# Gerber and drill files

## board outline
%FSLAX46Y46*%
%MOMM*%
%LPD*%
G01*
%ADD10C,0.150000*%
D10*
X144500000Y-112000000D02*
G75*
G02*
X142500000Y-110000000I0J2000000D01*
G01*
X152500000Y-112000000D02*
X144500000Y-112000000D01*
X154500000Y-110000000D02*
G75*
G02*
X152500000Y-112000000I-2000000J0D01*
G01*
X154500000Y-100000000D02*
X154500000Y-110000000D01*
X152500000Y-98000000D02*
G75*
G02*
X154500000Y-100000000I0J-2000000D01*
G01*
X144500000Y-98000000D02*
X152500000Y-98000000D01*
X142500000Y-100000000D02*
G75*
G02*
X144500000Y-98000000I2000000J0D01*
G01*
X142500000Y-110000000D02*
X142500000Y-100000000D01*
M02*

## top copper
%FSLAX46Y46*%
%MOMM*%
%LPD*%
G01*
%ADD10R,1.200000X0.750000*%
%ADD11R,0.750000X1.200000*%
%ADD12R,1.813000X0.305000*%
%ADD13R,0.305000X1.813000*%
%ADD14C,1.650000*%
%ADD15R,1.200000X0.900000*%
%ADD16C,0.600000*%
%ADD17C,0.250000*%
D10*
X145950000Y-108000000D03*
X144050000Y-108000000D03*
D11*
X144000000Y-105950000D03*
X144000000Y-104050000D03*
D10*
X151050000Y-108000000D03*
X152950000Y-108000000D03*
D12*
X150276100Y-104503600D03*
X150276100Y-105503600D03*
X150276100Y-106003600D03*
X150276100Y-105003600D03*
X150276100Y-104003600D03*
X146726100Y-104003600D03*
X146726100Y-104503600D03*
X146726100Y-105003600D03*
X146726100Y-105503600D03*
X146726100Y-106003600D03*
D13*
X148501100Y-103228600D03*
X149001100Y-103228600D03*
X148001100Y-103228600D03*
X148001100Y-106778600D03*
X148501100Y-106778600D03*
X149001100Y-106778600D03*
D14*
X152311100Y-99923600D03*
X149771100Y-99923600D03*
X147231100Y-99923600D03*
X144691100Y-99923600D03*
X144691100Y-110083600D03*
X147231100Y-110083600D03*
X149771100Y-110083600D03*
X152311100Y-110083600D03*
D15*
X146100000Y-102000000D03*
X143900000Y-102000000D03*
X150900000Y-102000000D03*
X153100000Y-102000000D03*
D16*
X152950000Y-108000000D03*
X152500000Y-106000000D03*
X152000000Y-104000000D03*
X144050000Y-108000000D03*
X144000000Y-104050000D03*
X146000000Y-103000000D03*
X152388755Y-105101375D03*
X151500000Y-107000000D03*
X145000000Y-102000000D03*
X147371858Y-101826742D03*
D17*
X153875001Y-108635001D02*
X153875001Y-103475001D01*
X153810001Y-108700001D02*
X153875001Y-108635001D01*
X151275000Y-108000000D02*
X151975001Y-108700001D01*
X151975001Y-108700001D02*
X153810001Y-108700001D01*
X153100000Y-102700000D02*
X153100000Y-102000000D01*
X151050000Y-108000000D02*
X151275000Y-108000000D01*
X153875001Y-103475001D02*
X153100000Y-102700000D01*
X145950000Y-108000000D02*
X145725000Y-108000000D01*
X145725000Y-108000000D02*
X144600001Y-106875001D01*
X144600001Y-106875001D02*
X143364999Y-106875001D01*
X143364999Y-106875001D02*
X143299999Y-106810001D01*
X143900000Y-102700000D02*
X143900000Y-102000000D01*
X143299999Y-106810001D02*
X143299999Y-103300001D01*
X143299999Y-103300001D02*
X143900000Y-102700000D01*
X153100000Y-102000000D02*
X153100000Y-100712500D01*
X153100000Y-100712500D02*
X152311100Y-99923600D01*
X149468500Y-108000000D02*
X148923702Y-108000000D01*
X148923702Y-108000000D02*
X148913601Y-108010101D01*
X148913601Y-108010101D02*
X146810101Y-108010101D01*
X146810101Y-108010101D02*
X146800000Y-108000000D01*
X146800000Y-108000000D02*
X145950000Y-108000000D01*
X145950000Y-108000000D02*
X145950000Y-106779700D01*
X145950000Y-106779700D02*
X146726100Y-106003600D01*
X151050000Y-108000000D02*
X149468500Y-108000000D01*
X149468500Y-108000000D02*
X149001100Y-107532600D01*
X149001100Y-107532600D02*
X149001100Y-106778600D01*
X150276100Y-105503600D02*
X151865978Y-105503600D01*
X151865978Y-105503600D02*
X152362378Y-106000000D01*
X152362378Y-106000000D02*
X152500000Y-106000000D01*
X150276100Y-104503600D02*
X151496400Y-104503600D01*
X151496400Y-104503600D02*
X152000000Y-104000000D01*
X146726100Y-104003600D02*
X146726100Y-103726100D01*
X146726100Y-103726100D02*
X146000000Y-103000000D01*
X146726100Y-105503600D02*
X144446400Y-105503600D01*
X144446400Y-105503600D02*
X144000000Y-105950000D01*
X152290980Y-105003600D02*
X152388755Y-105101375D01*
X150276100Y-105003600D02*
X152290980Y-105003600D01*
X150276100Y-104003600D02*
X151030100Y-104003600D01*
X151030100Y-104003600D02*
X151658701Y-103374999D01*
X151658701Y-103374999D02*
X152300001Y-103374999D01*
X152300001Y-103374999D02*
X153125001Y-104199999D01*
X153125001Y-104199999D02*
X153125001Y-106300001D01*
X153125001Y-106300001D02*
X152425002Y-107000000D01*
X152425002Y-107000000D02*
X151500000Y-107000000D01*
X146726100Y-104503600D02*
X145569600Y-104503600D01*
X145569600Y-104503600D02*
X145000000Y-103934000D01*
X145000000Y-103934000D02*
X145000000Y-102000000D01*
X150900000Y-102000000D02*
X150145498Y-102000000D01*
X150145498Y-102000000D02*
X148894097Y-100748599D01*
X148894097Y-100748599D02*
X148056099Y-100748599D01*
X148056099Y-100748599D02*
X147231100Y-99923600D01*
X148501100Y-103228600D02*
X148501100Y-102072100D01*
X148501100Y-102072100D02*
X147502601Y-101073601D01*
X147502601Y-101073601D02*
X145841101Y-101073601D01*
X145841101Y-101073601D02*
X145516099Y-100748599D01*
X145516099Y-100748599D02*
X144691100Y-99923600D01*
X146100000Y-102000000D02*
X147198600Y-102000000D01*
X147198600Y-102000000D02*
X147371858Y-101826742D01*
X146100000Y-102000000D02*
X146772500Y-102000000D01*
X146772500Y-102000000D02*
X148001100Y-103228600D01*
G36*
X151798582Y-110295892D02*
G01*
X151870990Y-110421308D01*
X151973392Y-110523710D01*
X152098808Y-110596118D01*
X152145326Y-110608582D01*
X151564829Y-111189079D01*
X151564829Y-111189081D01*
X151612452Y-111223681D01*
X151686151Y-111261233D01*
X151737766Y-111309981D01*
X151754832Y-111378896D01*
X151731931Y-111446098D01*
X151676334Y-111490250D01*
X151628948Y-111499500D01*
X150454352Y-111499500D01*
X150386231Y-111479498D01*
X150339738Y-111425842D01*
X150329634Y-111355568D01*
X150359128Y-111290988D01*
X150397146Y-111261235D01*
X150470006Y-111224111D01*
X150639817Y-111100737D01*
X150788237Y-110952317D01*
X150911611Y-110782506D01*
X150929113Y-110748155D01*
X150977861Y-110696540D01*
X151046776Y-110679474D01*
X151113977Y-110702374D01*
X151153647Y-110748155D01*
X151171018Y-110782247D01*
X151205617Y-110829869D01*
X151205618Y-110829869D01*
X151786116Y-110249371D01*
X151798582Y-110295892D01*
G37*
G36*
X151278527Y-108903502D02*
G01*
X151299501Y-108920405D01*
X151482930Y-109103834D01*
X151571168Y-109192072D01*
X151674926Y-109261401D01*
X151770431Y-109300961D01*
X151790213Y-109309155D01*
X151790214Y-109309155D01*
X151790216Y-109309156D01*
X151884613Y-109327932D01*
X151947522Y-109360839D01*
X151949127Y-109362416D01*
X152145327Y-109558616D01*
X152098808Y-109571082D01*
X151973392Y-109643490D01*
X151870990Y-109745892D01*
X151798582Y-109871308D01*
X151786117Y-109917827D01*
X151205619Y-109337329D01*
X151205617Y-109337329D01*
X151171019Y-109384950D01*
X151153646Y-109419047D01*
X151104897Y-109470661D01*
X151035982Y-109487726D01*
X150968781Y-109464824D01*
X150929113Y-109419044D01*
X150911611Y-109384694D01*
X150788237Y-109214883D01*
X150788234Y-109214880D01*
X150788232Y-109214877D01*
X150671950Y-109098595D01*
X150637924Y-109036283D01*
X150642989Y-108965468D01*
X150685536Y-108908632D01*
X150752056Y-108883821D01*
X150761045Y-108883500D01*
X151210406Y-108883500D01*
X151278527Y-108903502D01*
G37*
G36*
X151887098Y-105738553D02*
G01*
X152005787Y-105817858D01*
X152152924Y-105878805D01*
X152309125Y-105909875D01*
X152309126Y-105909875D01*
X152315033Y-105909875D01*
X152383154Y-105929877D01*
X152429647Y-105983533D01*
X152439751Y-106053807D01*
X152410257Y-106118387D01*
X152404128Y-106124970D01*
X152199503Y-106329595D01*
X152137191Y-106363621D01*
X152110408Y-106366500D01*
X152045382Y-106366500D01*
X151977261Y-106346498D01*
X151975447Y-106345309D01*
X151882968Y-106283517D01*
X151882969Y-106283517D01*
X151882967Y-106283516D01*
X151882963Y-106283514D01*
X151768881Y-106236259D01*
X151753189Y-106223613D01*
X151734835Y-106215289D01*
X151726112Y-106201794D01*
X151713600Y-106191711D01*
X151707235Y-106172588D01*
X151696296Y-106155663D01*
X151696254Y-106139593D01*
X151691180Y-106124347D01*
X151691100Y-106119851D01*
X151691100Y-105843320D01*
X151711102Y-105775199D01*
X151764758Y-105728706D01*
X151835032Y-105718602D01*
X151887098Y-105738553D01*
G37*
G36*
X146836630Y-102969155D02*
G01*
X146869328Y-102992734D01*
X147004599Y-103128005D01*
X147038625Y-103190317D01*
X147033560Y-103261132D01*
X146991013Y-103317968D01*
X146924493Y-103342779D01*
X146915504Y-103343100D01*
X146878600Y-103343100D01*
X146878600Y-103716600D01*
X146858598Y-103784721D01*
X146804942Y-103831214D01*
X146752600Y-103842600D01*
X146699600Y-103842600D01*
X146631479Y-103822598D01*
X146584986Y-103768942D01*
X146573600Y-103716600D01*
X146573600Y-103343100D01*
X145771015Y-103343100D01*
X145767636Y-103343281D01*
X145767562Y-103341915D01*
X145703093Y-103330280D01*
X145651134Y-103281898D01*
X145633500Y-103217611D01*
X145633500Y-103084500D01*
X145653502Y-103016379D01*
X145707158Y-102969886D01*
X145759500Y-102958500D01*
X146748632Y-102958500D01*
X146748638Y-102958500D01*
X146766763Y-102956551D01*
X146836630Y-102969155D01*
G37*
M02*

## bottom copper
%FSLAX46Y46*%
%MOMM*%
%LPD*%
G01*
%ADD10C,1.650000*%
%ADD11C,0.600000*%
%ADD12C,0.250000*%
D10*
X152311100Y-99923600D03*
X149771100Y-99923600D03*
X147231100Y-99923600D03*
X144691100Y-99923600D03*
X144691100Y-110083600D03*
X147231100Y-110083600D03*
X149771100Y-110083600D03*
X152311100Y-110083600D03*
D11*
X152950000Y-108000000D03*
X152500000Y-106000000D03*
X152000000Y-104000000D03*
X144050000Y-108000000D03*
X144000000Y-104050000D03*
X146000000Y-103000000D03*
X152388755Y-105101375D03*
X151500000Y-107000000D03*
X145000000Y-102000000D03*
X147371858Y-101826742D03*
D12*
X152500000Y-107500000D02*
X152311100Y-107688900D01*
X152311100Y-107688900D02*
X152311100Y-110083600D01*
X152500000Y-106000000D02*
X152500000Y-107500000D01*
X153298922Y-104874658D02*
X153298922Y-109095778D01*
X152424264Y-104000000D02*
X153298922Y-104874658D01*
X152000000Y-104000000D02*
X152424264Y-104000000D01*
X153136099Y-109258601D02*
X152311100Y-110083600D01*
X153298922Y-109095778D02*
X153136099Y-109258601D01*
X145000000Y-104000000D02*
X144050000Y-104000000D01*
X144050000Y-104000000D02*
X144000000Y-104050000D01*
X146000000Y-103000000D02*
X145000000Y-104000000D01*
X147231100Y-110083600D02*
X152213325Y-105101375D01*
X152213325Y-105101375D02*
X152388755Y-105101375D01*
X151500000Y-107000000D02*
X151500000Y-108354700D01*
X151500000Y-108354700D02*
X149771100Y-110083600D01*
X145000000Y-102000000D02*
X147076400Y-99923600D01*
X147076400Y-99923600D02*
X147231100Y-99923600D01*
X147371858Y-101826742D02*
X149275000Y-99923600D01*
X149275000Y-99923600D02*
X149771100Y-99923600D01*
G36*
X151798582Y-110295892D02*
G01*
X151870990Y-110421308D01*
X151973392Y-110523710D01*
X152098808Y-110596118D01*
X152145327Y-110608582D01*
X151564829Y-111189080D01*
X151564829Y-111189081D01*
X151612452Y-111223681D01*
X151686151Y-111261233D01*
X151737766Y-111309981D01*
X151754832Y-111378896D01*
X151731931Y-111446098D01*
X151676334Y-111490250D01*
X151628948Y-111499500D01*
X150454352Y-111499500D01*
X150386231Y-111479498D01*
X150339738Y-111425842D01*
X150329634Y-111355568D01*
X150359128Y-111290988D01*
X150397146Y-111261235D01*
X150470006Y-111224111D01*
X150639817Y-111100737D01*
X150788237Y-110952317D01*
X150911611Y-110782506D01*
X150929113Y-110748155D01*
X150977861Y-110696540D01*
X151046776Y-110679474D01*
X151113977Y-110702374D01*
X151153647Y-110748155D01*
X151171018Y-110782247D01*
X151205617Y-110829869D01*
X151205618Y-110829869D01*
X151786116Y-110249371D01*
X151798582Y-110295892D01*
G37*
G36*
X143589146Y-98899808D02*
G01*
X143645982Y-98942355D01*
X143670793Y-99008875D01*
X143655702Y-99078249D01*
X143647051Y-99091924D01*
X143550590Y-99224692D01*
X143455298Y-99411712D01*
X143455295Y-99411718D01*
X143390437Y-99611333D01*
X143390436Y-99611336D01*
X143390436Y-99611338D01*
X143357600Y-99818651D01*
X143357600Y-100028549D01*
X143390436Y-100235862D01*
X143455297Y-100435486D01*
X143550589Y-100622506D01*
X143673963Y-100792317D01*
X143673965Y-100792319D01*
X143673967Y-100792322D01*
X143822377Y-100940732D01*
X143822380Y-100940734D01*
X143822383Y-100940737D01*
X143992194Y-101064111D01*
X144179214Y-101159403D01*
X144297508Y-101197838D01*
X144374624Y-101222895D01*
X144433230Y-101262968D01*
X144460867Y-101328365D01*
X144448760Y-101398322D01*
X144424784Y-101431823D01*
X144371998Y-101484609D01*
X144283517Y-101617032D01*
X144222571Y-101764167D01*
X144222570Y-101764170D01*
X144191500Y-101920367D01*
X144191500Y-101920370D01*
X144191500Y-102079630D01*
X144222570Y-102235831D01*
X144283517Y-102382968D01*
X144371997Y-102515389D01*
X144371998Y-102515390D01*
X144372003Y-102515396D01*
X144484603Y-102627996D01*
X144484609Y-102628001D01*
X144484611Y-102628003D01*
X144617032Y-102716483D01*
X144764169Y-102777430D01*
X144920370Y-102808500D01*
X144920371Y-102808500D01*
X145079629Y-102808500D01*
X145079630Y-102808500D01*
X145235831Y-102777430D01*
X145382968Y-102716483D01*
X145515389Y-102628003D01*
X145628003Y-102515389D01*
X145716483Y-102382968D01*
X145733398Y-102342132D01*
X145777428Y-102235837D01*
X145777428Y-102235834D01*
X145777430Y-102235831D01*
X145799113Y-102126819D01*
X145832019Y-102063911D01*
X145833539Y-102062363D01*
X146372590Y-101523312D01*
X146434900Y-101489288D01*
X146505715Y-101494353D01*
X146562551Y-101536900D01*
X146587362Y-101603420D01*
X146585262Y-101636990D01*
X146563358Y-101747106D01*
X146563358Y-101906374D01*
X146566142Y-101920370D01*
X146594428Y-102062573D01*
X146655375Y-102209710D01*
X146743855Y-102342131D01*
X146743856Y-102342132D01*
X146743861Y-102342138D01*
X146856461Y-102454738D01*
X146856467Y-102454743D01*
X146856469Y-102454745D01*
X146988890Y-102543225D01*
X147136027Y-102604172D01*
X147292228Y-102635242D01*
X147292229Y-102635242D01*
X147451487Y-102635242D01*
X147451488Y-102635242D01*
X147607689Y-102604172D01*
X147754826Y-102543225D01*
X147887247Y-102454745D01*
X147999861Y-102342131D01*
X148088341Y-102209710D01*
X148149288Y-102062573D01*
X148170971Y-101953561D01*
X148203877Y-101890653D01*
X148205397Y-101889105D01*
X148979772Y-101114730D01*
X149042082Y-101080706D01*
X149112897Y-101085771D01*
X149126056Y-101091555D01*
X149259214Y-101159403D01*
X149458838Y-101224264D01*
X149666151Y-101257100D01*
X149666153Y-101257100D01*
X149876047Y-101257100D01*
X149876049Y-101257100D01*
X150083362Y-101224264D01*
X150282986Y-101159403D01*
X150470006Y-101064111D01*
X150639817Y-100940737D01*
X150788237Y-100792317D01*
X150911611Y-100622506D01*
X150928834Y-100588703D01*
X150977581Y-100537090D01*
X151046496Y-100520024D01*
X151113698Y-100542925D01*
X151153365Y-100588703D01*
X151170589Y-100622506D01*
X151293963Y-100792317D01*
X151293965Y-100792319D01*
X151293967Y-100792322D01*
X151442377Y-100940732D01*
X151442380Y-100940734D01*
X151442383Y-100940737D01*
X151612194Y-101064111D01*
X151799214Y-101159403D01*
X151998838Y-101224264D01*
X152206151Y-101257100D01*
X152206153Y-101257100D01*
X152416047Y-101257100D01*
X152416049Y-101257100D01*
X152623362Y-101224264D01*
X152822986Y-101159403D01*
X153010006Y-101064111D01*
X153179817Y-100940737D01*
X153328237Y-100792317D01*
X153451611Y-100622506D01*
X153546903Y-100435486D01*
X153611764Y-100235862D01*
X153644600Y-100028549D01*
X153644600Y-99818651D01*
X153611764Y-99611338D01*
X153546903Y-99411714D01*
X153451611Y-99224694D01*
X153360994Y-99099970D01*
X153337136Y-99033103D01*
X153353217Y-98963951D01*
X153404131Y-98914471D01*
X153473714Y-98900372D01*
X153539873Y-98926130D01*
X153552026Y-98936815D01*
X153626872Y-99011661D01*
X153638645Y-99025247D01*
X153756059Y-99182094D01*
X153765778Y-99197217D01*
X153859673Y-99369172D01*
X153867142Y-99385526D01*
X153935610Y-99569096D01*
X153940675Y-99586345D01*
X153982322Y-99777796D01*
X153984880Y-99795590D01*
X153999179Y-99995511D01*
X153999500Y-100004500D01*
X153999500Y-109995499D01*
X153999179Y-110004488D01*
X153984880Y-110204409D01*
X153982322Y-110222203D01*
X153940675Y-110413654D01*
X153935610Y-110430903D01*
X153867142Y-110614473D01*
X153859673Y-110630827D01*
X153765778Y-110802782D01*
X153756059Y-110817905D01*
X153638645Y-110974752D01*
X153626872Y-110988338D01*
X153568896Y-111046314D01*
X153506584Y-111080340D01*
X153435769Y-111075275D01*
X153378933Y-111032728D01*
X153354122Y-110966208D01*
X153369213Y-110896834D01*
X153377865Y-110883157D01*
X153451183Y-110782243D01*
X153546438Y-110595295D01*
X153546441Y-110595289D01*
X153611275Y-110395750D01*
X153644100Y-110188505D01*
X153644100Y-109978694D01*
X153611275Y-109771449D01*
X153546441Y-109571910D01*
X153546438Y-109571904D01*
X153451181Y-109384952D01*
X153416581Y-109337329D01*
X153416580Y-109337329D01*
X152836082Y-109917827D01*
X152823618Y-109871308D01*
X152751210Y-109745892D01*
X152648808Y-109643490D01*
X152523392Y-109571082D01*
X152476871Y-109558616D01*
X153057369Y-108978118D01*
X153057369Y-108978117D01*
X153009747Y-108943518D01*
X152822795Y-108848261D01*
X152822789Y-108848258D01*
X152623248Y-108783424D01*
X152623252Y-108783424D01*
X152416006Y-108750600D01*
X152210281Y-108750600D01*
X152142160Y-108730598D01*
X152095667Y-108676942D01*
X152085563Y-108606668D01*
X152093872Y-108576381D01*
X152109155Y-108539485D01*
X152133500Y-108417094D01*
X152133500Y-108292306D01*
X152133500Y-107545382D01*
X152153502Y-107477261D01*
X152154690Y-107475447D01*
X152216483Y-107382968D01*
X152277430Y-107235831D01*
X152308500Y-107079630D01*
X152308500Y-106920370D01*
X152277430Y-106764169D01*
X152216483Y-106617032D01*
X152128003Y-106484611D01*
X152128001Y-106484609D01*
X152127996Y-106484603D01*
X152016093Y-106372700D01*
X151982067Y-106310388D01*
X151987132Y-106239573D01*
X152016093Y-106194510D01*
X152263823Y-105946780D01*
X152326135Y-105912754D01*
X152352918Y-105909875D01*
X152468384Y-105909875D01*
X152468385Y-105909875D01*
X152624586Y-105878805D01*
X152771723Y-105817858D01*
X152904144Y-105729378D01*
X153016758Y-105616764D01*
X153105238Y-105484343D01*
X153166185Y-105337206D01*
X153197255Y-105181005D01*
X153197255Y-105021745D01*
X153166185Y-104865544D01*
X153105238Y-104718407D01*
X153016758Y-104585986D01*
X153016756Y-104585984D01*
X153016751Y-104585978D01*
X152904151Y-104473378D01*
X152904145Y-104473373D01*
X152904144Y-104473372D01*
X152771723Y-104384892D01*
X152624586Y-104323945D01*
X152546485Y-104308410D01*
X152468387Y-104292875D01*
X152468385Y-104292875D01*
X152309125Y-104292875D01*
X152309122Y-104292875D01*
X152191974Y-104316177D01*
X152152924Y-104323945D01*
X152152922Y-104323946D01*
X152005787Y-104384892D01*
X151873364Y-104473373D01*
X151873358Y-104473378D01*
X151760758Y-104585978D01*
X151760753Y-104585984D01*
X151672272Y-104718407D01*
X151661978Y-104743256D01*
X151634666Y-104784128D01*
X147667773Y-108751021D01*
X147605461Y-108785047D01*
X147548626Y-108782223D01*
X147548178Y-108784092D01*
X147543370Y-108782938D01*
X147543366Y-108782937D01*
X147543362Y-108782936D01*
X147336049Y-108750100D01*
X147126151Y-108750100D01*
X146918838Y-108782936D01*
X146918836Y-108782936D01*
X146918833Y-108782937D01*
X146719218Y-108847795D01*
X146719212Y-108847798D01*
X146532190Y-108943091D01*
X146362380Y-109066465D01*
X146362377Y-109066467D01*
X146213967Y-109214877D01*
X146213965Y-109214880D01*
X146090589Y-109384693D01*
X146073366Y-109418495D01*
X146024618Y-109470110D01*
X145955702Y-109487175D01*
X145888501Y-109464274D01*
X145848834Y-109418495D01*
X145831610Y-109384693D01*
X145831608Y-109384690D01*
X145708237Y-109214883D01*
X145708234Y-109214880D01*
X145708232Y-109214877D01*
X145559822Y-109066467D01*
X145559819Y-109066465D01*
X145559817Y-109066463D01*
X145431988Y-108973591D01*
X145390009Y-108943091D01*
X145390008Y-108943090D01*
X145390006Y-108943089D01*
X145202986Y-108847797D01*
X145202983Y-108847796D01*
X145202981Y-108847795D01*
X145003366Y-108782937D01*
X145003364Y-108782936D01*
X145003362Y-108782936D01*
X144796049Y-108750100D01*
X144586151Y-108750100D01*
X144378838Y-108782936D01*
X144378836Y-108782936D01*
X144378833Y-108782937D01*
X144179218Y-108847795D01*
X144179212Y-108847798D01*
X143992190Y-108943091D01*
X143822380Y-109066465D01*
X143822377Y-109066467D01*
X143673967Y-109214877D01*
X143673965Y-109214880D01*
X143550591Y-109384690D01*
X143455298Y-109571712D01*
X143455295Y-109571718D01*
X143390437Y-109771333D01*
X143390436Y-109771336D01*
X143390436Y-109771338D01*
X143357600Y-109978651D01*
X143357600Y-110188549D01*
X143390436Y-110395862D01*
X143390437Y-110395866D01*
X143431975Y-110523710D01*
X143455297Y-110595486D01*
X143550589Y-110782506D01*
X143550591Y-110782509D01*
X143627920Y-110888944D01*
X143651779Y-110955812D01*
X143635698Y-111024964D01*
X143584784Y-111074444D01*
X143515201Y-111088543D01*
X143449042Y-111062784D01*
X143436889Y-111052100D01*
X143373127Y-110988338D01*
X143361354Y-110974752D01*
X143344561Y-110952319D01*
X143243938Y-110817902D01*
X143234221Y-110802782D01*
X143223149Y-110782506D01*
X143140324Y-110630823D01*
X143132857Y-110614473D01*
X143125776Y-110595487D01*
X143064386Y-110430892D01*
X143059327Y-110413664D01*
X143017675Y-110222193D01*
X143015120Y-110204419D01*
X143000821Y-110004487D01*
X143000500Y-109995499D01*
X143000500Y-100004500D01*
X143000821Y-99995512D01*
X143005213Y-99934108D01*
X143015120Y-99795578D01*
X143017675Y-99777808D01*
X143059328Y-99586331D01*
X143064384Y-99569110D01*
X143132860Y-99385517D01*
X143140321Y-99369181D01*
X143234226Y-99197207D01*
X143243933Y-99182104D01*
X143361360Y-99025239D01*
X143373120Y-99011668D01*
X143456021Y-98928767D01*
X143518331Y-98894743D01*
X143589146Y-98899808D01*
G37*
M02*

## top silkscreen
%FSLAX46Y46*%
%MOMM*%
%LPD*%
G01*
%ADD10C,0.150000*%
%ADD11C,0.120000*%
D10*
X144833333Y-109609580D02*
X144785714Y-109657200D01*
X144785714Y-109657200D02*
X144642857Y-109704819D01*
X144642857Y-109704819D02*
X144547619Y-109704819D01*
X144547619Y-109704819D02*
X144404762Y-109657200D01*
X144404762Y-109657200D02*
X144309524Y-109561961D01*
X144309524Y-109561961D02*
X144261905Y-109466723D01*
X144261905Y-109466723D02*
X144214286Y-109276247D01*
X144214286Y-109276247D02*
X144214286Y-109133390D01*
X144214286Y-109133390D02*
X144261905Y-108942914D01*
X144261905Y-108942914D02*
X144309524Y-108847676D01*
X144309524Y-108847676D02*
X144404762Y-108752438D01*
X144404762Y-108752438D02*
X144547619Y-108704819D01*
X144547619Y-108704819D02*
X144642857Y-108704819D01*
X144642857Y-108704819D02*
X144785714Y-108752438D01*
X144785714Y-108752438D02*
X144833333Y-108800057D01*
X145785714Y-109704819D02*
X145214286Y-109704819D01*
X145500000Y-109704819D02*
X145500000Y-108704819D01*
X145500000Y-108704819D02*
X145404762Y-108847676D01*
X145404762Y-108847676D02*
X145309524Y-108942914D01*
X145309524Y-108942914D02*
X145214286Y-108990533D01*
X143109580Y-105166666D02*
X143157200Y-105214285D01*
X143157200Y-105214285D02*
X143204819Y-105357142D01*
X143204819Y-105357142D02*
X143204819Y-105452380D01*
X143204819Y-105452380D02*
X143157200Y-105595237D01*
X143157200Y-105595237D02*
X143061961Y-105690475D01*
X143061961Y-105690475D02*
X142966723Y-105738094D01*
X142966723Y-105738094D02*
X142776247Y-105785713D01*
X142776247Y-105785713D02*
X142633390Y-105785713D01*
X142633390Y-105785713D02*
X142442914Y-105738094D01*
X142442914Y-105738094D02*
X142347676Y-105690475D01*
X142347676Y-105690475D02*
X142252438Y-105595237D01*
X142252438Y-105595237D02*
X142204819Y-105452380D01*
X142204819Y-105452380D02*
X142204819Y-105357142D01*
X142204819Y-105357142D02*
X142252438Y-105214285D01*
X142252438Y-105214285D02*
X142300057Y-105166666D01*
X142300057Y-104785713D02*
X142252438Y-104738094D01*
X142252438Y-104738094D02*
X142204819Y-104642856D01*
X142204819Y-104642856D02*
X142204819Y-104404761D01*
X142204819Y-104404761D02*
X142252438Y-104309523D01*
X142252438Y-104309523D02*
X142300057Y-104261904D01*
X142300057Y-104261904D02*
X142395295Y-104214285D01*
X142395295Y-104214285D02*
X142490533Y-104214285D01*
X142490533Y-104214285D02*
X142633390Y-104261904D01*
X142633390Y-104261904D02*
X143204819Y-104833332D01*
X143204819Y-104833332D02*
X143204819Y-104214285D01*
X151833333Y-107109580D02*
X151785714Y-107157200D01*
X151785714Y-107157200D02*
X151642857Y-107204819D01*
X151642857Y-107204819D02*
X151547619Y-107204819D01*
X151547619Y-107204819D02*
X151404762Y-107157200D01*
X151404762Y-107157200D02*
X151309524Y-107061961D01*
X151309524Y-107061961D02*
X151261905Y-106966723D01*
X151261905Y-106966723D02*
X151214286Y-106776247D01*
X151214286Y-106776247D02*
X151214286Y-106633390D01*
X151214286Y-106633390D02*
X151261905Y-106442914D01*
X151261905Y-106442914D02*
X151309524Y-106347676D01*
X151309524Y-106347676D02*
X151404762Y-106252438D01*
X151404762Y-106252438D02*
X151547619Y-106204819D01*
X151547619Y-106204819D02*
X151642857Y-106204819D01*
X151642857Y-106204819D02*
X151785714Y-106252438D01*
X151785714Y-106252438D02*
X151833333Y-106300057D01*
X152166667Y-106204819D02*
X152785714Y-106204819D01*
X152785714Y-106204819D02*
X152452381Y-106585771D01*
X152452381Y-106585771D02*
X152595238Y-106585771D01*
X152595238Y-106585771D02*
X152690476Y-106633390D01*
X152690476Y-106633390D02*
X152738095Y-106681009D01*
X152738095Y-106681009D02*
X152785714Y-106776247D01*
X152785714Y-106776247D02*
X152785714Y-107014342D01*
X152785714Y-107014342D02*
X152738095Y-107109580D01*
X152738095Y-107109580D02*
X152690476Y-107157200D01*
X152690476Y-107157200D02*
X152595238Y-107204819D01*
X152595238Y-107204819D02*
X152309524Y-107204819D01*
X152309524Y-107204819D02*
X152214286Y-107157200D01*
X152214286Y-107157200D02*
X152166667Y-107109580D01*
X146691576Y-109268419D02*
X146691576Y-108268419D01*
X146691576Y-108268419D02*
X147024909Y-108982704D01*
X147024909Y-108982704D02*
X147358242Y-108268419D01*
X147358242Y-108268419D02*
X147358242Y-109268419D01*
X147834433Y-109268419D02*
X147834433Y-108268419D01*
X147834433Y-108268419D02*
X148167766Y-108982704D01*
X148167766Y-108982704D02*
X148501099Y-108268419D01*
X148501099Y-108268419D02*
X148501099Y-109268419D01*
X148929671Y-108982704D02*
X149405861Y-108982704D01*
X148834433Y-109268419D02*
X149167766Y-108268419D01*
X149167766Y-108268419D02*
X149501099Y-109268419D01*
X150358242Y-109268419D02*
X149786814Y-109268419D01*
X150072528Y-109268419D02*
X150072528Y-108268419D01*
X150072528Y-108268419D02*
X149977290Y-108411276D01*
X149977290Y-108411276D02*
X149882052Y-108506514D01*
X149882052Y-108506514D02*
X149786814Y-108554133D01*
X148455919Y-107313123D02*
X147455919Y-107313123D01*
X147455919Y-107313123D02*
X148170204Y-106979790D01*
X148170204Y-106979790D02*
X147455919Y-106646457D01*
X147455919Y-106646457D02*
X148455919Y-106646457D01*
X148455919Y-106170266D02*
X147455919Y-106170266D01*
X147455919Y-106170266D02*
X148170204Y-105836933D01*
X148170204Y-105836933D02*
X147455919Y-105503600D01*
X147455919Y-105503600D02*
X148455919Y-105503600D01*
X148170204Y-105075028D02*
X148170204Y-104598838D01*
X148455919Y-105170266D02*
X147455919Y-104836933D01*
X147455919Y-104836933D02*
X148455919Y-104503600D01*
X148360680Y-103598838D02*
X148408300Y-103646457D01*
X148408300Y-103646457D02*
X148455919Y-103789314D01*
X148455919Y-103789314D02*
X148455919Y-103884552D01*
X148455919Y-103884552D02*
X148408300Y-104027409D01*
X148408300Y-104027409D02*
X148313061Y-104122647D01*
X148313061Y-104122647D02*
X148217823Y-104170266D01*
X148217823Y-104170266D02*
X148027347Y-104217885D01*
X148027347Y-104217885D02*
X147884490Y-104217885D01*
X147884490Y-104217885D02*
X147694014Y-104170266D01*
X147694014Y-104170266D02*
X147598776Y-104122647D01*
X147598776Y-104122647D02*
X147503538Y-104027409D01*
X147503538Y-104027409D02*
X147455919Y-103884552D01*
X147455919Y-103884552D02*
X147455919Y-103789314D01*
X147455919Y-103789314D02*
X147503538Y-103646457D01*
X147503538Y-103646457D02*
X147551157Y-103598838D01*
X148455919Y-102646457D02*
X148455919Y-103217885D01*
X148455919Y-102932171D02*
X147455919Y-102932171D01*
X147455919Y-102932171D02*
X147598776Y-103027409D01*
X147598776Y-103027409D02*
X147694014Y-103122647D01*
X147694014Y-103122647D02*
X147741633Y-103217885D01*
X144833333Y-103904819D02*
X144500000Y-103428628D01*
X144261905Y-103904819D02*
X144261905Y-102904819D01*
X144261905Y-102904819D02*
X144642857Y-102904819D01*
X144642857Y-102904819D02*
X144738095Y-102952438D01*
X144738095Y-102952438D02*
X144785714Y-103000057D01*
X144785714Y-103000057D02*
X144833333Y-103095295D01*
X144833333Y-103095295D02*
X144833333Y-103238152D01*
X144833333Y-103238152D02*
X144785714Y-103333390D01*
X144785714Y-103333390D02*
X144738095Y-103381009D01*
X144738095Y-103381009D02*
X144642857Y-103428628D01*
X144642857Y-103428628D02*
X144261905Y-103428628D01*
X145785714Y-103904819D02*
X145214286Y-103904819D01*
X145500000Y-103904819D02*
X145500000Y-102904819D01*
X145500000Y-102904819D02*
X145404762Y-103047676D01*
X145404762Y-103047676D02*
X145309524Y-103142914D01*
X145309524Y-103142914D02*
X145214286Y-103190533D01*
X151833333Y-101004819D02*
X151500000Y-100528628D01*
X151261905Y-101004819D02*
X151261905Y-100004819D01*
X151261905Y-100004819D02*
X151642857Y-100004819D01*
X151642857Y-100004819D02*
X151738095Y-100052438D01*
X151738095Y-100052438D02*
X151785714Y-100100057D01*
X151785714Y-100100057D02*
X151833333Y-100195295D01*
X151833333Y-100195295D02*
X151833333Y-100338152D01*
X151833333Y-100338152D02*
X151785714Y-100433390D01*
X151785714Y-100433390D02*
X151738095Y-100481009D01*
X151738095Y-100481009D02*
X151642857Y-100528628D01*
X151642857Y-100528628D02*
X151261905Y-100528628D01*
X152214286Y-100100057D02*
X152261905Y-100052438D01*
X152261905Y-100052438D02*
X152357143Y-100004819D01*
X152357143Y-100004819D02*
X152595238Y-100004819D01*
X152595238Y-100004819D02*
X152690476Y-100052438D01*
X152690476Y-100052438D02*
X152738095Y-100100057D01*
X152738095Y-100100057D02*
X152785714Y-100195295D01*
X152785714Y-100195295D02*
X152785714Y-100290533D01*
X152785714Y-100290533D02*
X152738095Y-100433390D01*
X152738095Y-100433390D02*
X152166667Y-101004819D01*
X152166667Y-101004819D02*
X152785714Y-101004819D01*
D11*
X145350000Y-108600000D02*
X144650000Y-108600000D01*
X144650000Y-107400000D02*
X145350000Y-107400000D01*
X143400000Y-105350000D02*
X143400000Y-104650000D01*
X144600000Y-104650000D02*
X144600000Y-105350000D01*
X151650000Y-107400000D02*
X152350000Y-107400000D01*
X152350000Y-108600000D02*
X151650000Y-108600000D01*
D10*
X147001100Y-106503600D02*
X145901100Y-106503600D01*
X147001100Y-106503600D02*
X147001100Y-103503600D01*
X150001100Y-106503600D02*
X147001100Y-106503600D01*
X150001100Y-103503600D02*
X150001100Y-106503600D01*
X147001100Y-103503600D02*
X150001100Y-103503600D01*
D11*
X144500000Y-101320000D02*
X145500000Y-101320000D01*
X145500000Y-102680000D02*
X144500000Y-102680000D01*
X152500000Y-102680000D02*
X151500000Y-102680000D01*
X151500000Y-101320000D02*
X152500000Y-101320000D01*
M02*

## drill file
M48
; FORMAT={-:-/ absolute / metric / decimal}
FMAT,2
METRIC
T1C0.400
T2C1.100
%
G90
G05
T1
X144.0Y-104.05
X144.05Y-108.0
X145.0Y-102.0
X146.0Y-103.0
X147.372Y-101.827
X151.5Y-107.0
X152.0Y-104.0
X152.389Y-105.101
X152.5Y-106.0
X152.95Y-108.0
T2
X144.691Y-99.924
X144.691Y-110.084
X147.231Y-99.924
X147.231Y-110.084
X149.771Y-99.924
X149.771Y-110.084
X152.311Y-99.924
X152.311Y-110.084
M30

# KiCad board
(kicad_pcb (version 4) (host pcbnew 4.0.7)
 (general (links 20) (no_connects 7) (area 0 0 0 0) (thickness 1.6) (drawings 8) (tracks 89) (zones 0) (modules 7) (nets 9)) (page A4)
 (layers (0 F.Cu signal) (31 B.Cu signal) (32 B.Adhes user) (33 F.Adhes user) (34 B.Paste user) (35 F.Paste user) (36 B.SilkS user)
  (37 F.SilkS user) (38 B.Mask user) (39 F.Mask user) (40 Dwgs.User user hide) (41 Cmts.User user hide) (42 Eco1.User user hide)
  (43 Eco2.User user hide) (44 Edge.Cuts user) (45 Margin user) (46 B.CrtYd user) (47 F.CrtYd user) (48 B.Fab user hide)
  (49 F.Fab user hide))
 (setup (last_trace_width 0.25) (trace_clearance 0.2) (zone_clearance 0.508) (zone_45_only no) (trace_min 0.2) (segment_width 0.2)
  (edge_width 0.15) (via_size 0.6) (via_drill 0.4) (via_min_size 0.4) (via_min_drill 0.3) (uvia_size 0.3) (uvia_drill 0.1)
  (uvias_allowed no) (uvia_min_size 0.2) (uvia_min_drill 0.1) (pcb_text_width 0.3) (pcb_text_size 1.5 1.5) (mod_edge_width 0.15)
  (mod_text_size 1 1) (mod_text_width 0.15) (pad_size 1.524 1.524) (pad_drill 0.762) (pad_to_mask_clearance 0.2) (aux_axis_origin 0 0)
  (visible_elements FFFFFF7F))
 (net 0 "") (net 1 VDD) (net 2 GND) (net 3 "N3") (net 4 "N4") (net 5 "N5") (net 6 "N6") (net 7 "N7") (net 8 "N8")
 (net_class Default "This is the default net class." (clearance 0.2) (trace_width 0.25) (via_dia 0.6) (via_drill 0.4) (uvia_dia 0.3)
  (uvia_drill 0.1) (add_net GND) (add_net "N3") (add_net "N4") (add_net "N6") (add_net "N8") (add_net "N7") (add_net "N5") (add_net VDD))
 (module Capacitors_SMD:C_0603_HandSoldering (layer F.Cu) (at 145 108 180)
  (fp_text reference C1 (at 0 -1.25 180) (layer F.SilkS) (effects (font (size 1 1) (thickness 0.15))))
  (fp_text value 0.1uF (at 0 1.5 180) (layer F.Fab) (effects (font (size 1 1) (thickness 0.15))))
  (fp_line (start -0.35 -0.6) (end 0.35 -0.6) (layer F.SilkS) (width 0.12))
  (fp_line (start 0.35 0.6) (end -0.35 0.6) (layer F.SilkS) (width 0.12))
  (pad 1 smd rect (at -0.95 0 180) (size 1.2 0.75) (layers F.Cu F.Paste F.Mask) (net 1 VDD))
  (pad 2 smd rect (at 0.95 0 180) (size 1.2 0.75) (layers F.Cu F.Paste F.Mask) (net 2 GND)))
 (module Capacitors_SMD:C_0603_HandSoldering (layer F.Cu) (at 144 105 90)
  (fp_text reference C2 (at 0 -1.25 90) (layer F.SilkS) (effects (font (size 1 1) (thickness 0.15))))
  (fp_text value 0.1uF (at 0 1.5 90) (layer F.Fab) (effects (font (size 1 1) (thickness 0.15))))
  (fp_line (start -0.35 -0.6) (end 0.35 -0.6) (layer F.SilkS) (width 0.12))
  (fp_line (start 0.35 0.6) (end -0.35 0.6) (layer F.SilkS) (width 0.12))
  (pad 1 smd rect (at -0.95 0 90) (size 1.2 0.75) (layers F.Cu F.Paste F.Mask) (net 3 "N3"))
  (pad 2 smd rect (at 0.95 0 90) (size 1.2 0.75) (layers F.Cu F.Paste F.Mask) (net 2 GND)))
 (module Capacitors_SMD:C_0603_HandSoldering (layer F.Cu) (at 152 108)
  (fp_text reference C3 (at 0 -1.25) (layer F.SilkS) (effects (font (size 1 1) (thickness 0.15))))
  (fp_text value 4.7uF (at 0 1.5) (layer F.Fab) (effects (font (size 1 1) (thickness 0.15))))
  (fp_line (start -0.35 -0.6) (end 0.35 -0.6) (layer F.SilkS) (width 0.12))
  (fp_line (start 0.35 0.6) (end -0.35 0.6) (layer F.SilkS) (width 0.12))
  (pad 1 smd rect (at -0.95 0) (size 1.2 0.75) (layers F.Cu F.Paste F.Mask) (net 1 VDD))
  (pad 2 smd rect (at 0.95 0) (size 1.2 0.75) (layers F.Cu F.Paste F.Mask) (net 2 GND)))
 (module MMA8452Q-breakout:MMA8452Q (layer F.Cu) (at 148.5011 105.0036)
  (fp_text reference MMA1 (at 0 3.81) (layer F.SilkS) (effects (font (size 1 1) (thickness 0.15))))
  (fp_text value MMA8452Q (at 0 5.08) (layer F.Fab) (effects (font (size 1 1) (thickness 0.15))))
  (fp_line (start -1.5 1.5) (end -2.6 1.5) (layer F.SilkS) (width 0.15))
  (fp_line (start -1.5 1.5) (end -1.5 -1.5) (layer F.SilkS) (width 0.15))
  (fp_line (start 1.5 1.5) (end -1.5 1.5) (layer F.SilkS) (width 0.15))
  (fp_line (start 1.5 -1.5) (end 1.5 1.5) (layer F.SilkS) (width 0.15))
  (fp_line (start -1.5 -1.5) (end 1.5 -1.5) (layer F.SilkS) (width 0.15))
  (pad 10 smd rect (at 1.775 -0.5) (size 1.813 0.305) (layers F.Cu F.Paste F.Mask) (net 2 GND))
  (pad 12 smd rect (at 1.775 0.5) (size 1.813 0.305) (layers F.Cu F.Paste F.Mask) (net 2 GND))
  (pad 13 smd rect (at 1.775 1) (size 1.813 0.305) (layers F.Cu F.Paste F.Mask))
  (pad 11 smd rect (at 1.775 0) (size 1.813 0.305) (layers F.Cu F.Paste F.Mask) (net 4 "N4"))
  (pad 9 smd rect (at 1.775 -1) (size 1.813 0.305) (layers F.Cu F.Paste F.Mask) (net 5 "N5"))
  (pad 5 smd rect (at -1.775 -1) (size 1.813 0.305) (layers F.Cu F.Paste F.Mask) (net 2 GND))
  (pad 4 smd rect (at -1.775 -0.5) (size 1.813 0.305) (layers F.Cu F.Paste F.Mask) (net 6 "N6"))
  (pad 3 smd rect (at -1.775 0) (size 1.813 0.305) (layers F.Cu F.Paste F.Mask))
  (pad 2 smd rect (at -1.775 0.5) (size 1.813 0.305) (layers F.Cu F.Paste F.Mask) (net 3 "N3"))
  (pad 1 smd rect (at -1.775 1) (size 1.813 0.305) (layers F.Cu F.Paste F.Mask) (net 1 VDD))
  (pad 7 smd rect (at 0 -1.775 90) (size 1.813 0.305) (layers F.Cu F.Paste F.Mask) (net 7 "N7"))
  (pad 8 smd rect (at 0.5 -1.775 90) (size 1.813 0.305) (layers F.Cu F.Paste F.Mask))
  (pad 6 smd rect (at -0.5 -1.775 90) (size 1.813 0.305) (layers F.Cu F.Paste F.Mask) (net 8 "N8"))
  (pad 16 smd rect (at -0.5 1.775 90) (size 1.813 0.305) (layers F.Cu F.Paste F.Mask))
  (pad 15 smd rect (at 0 1.775 90) (size 1.813 0.305) (layers F.Cu F.Paste F.Mask))
  (pad 14 smd rect (at 0.5 1.775 90) (size 1.813 0.305) (layers F.Cu F.Paste F.Mask) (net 1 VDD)))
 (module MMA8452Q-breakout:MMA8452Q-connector (layer F.Cu) (at 148.5011 105.0036 270)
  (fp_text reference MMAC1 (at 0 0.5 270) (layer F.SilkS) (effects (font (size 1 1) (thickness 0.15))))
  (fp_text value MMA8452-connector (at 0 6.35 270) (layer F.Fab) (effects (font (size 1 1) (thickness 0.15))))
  (pad 1 thru_hole circle (at -5.08 -3.81 270) (size 1.65 1.65) (drill 1.1) (layers *.Cu *.Mask) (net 1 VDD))
  (pad 2 thru_hole circle (at -5.08 -1.27 270) (size 1.65 1.65) (drill 1.1) (layers *.Cu *.Mask) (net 8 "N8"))
  (pad 3 thru_hole circle (at -5.08 1.27 270) (size 1.65 1.65) (drill 1.1) (layers *.Cu *.Mask) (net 6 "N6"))
  (pad 4 thru_hole circle (at -5.08 3.81 270) (size 1.65 1.65) (drill 1.1) (layers *.Cu *.Mask) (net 7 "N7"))
  (pad 5 thru_hole circle (at 5.08 3.81 270) (size 1.65 1.65) (drill 1.1) (layers *.Cu *.Mask))
  (pad 6 thru_hole circle (at 5.08 1.27 270) (size 1.65 1.65) (drill 1.1) (layers *.Cu *.Mask) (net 4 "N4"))
  (pad 7 thru_hole circle (at 5.08 -1.27 270) (size 1.65 1.65) (drill 1.1) (layers *.Cu *.Mask) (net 5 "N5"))
  (pad 8 thru_hole circle (at 5.08 -3.81 270) (size 1.65 1.65) (drill 1.1) (layers *.Cu *.Mask) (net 2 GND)))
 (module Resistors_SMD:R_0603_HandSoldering (layer F.Cu) (at 145 102 180)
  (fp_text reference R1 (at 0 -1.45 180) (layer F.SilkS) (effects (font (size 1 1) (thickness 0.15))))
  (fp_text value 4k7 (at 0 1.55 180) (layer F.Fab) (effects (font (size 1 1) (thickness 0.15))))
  (fp_line (start 0.5 0.68) (end -0.5 0.68) (layer F.SilkS) (width 0.12))
  (fp_line (start -0.5 -0.68) (end 0.5 -0.68) (layer F.SilkS) (width 0.12))
  (pad 1 smd rect (at -1.1 0 180) (size 1.2 0.9) (layers F.Cu F.Paste F.Mask) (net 8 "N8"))
  (pad 2 smd rect (at 1.1 0 180) (size 1.2 0.9) (layers F.Cu F.Paste F.Mask) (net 1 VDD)))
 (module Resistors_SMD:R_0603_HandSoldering (layer F.Cu) (at 152 102)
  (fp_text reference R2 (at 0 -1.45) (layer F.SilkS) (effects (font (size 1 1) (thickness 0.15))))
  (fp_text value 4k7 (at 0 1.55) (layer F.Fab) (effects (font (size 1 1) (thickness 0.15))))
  (fp_line (start 0.5 0.68) (end -0.5 0.68) (layer F.SilkS) (width 0.12))
  (fp_line (start -0.5 -0.68) (end 0.5 -0.68) (layer F.SilkS) (width 0.12))
  (pad 1 smd rect (at -1.1 0) (size 1.2 0.9) (layers F.Cu F.Paste F.Mask) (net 6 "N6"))
  (pad 2 smd rect (at 1.1 0) (size 1.2 0.9) (layers F.Cu F.Paste F.Mask) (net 1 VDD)))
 (gr_arc (start 144.5 110) (end 144.5 112) (angle 90) (layer Edge.Cuts) (width 0.15))
 (gr_line (start 152.5 112) (end 144.5 112) (layer Edge.Cuts) (width 0.15))
 (gr_arc (start 152.5 110) (end 154.5 110) (angle 90) (layer Edge.Cuts) (width 0.15))
 (gr_line (start 154.5 100) (end 154.5 110) (layer Edge.Cuts) (width 0.15))
 (gr_arc (start 152.5 100) (end 152.5 98) (angle 90) (layer Edge.Cuts) (width 0.15))
 (gr_line (start 144.5 98) (end 152.5 98) (layer Edge.Cuts) (width 0.15))
 (gr_arc (start 144.5 100) (end 142.5 100) (angle 90) (layer Edge.Cuts) (width 0.15))
 (gr_line (start 142.5 110) (end 142.5 100) (layer Edge.Cuts) (width 0.15))
 (segment (start 153.875001 108.635001) (end 153.875001 103.475001) (width 0.25) (layer F.Cu) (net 1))
 (segment (start 153.810001 108.700001) (end 153.875001 108.635001) (width 0.25) (layer F.Cu) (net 1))
 (segment (start 151.275 108) (end 151.975001 108.700001) (width 0.25) (layer F.Cu) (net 1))
 (segment (start 151.975001 108.700001) (end 153.810001 108.700001) (width 0.25) (layer F.Cu) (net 1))
 (segment (start 153.1 102.7) (end 153.1 102) (width 0.25) (layer F.Cu) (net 1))
 (segment (start 151.05 108) (end 151.275 108) (width 0.25) (layer F.Cu) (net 1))
 (segment (start 153.875001 103.475001) (end 153.1 102.7) (width 0.25) (layer F.Cu) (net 1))
 (segment (start 145.95 108) (end 145.725 108) (width 0.25) (layer F.Cu) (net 1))
 (segment (start 145.725 108) (end 144.600001 106.875001) (width 0.25) (layer F.Cu) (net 1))
 (segment (start 144.600001 106.875001) (end 143.364999 106.875001) (width 0.25) (layer F.Cu) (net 1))
 (segment (start 143.364999 106.875001) (end 143.299999 106.810001) (width 0.25) (layer F.Cu) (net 1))
 (segment (start 143.9 102.7) (end 143.9 102) (width 0.25) (layer F.Cu) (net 1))
 (segment (start 143.299999 106.810001) (end 143.299999 103.300001) (width 0.25) (layer F.Cu) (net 1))
 (segment (start 143.299999 103.300001) (end 143.9 102.7) (width 0.25) (layer F.Cu) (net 1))
 (segment (start 153.1 102) (end 153.1 100.7125) (width 0.25) (layer F.Cu) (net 1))
 (segment (start 153.1 100.7125) (end 152.3111 99.9236) (width 0.25) (layer F.Cu) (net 1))
 (segment (start 149.4685 108) (end 148.923702 108) (width 0.25) (layer F.Cu) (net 1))
 (segment (start 148.923702 108) (end 148.913601 108.010101) (width 0.25) (layer F.Cu) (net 1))
 (segment (start 148.913601 108.010101) (end 146.810101 108.010101) (width 0.25) (layer F.Cu) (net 1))
 (segment (start 146.810101 108.010101) (end 146.8 108) (width 0.25) (layer F.Cu) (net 1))
 (segment (start 146.8 108) (end 145.95 108) (width 0.25) (layer F.Cu) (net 1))
 (segment (start 145.95 108) (end 145.95 106.7797) (width 0.25) (layer F.Cu) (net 1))
 (segment (start 145.95 106.7797) (end 146.7261 106.0036) (width 0.25) (layer F.Cu) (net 1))
 (segment (start 151.05 108) (end 149.4685 108) (width 0.25) (layer F.Cu) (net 1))
 (segment (start 149.4685 108) (end 149.0011 107.5326) (width 0.25) (layer F.Cu) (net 1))
 (segment (start 149.0011 107.5326) (end 149.0011 106.7786) (width 0.25) (layer F.Cu) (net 1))
 (via (at 152.95 108) (size 0.6) (drill 0.4) (layers F.Cu B.Cu) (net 2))
 (segment (start 152.5 107.5) (end 152.3111 107.6889) (width 0.25) (layer B.Cu) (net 2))
 (segment (start 152.3111 107.6889) (end 152.3111 110.0836) (width 0.25) (layer B.Cu) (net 2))
 (segment (start 152.5 106) (end 152.5 107.5) (width 0.25) (layer B.Cu) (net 2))
 (segment (start 150.2761 105.5036) (end 151.865978 105.5036) (width 0.25) (layer F.Cu) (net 2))
 (segment (start 151.865978 105.5036) (end 152.362378 106) (width 0.25) (layer F.Cu) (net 2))
 (segment (start 152.362378 106) (end 152.5 106) (width 0.25) (layer F.Cu) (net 2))
 (via (at 152.5 106) (size 0.6) (drill 0.4) (layers F.Cu B.Cu) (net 2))
 (segment (start 153.298922 104.874658) (end 153.298922 109.095778) (width 0.25) (layer B.Cu) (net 2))
 (segment (start 152.424264 104) (end 153.298922 104.874658) (width 0.25) (layer B.Cu) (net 2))
 (segment (start 152 104) (end 152.424264 104) (width 0.25) (layer B.Cu) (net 2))
 (segment (start 153.136099 109.258601) (end 152.3111 110.0836) (width 0.25) (layer B.Cu) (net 2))
 (segment (start 153.298922 109.095778) (end 153.136099 109.258601) (width 0.25) (layer B.Cu) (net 2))
 (segment (start 150.2761 104.5036) (end 151.4964 104.5036) (width 0.25) (layer F.Cu) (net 2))
 (segment (start 151.4964 104.5036) (end 152 104) (width 0.25) (layer F.Cu) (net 2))
 (via (at 152 104) (size 0.6) (drill 0.4) (layers F.Cu B.Cu) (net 2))
 (via (at 144.05 108) (size 0.6) (drill 0.4) (layers F.Cu B.Cu) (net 2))
 (segment (start 145 104) (end 144.05 104) (width 0.25) (layer B.Cu) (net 2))
 (segment (start 144.05 104) (end 144 104.05) (width 0.25) (layer B.Cu) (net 2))
 (via (at 144 104.05) (size 0.6) (drill 0.4) (layers F.Cu B.Cu) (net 2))
 (segment (start 146 103) (end 145 104) (width 0.25) (layer B.Cu) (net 2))
 (segment (start 146.7261 104.0036) (end 146.7261 103.7261) (width 0.25) (layer F.Cu) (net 2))
 (segment (start 146.7261 103.7261) (end 146 103) (width 0.25) (layer F.Cu) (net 2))
 (via (at 146 103) (size 0.6) (drill 0.4) (layers F.Cu B.Cu) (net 2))
 (segment (start 146.7261 105.5036) (end 144.4464 105.5036) (width 0.25) (layer F.Cu) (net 3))
 (segment (start 144.4464 105.5036) (end 144 105.95) (width 0.25) (layer F.Cu) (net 3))
 (segment (start 152.29098 105.0036) (end 152.388755 105.101375) (width 0.25) (layer F.Cu) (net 4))
 (via (at 152.388755 105.101375) (size 0.6) (drill 0.4) (layers F.Cu B.Cu) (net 4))
 (segment (start 147.2311 110.0836) (end 152.213325 105.101375) (width 0.25) (layer B.Cu) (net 4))
 (segment (start 152.213325 105.101375) (end 152.388755 105.101375) (width 0.25) (layer B.Cu) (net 4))
 (segment (start 150.2761 105.0036) (end 152.29098 105.0036) (width 0.25) (layer F.Cu) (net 4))
 (segment (start 151.5 107) (end 151.5 108.3547) (width 0.25) (layer B.Cu) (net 5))
 (segment (start 151.5 108.3547) (end 149.7711 110.0836) (width 0.25) (layer B.Cu) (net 5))
 (segment (start 150.2761 104.0036) (end 151.0301 104.0036) (width 0.25) (layer F.Cu) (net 5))
 (segment (start 151.0301 104.0036) (end 151.658701 103.374999) (width 0.25) (layer F.Cu) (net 5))
 (segment (start 151.658701 103.374999) (end 152.300001 103.374999) (width 0.25) (layer F.Cu) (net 5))
 (segment (start 152.300001 103.374999) (end 153.125001 104.199999) (width 0.25) (layer F.Cu) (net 5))
 (segment (start 153.125001 104.199999) (end 153.125001 106.300001) (width 0.25) (layer F.Cu) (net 5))
 (segment (start 153.125001 106.300001) (end 152.425002 107) (width 0.25) (layer F.Cu) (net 5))
 (segment (start 152.425002 107) (end 151.5 107) (width 0.25) (layer F.Cu) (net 5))
 (via (at 151.5 107) (size 0.6) (drill 0.4) (layers F.Cu B.Cu) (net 5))
 (segment (start 145 102) (end 147.0764 99.9236) (width 0.25) (layer B.Cu) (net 6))
 (segment (start 147.0764 99.9236) (end 147.2311 99.9236) (width 0.25) (layer B.Cu) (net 6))
 (segment (start 146.7261 104.5036) (end 145.5696 104.5036) (width 0.25) (layer F.Cu) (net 6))
 (segment (start 145.5696 104.5036) (end 145 103.934) (width 0.25) (layer F.Cu) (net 6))
 (segment (start 145 103.934) (end 145 102) (width 0.25) (layer F.Cu) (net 6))
 (via (at 145 102) (size 0.6) (drill 0.4) (layers F.Cu B.Cu) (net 6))
 (segment (start 150.9 102) (end 150.145498 102) (width 0.25) (layer F.Cu) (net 6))
 (segment (start 150.145498 102) (end 148.894097 100.748599) (width 0.25) (layer F.Cu) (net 6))
 (segment (start 148.894097 100.748599) (end 148.056099 100.748599) (width 0.25) (layer F.Cu) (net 6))
 (segment (start 148.056099 100.748599) (end 147.2311 99.9236) (width 0.25) (layer F.Cu) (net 6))
 (segment (start 148.5011 103.2286) (end 148.5011 102.0721) (width 0.25) (layer F.Cu) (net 7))
 (segment (start 148.5011 102.0721) (end 147.502601 101.073601) (width 0.25) (layer F.Cu) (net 7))
 (segment (start 147.502601 101.073601) (end 145.841101 101.073601) (width 0.25) (layer F.Cu) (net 7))
 (segment (start 145.841101 101.073601) (end 145.516099 100.748599) (width 0.25) (layer F.Cu) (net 7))
 (segment (start 145.516099 100.748599) (end 144.6911 99.9236) (width 0.25) (layer F.Cu) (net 7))
 (segment (start 147.371858 101.826742) (end 149.275 99.9236) (width 0.25) (layer B.Cu) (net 8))
 (segment (start 149.275 99.9236) (end 149.7711 99.9236) (width 0.25) (layer B.Cu) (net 8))
 (segment (start 146.1 102) (end 147.1986 102) (width 0.25) (layer F.Cu) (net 8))
 (segment (start 147.1986 102) (end 147.371858 101.826742) (width 0.25) (layer F.Cu) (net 8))
 (via (at 147.371858 101.826742) (size 0.6) (drill 0.4) (layers F.Cu B.Cu) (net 8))
 (segment (start 146.1 102) (end 146.7725 102) (width 0.25) (layer F.Cu) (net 8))
 (segment (start 146.7725 102) (end 148.0011 103.2286) (width 0.25) (layer F.Cu) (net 8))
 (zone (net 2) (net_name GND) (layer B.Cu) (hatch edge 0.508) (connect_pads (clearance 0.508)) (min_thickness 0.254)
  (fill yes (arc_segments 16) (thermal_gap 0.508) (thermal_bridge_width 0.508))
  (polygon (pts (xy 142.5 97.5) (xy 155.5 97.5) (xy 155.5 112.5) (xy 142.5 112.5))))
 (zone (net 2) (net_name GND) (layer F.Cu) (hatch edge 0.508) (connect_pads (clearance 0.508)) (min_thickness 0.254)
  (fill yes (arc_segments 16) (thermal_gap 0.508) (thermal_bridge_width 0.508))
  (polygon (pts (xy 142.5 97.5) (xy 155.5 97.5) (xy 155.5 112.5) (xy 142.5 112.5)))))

